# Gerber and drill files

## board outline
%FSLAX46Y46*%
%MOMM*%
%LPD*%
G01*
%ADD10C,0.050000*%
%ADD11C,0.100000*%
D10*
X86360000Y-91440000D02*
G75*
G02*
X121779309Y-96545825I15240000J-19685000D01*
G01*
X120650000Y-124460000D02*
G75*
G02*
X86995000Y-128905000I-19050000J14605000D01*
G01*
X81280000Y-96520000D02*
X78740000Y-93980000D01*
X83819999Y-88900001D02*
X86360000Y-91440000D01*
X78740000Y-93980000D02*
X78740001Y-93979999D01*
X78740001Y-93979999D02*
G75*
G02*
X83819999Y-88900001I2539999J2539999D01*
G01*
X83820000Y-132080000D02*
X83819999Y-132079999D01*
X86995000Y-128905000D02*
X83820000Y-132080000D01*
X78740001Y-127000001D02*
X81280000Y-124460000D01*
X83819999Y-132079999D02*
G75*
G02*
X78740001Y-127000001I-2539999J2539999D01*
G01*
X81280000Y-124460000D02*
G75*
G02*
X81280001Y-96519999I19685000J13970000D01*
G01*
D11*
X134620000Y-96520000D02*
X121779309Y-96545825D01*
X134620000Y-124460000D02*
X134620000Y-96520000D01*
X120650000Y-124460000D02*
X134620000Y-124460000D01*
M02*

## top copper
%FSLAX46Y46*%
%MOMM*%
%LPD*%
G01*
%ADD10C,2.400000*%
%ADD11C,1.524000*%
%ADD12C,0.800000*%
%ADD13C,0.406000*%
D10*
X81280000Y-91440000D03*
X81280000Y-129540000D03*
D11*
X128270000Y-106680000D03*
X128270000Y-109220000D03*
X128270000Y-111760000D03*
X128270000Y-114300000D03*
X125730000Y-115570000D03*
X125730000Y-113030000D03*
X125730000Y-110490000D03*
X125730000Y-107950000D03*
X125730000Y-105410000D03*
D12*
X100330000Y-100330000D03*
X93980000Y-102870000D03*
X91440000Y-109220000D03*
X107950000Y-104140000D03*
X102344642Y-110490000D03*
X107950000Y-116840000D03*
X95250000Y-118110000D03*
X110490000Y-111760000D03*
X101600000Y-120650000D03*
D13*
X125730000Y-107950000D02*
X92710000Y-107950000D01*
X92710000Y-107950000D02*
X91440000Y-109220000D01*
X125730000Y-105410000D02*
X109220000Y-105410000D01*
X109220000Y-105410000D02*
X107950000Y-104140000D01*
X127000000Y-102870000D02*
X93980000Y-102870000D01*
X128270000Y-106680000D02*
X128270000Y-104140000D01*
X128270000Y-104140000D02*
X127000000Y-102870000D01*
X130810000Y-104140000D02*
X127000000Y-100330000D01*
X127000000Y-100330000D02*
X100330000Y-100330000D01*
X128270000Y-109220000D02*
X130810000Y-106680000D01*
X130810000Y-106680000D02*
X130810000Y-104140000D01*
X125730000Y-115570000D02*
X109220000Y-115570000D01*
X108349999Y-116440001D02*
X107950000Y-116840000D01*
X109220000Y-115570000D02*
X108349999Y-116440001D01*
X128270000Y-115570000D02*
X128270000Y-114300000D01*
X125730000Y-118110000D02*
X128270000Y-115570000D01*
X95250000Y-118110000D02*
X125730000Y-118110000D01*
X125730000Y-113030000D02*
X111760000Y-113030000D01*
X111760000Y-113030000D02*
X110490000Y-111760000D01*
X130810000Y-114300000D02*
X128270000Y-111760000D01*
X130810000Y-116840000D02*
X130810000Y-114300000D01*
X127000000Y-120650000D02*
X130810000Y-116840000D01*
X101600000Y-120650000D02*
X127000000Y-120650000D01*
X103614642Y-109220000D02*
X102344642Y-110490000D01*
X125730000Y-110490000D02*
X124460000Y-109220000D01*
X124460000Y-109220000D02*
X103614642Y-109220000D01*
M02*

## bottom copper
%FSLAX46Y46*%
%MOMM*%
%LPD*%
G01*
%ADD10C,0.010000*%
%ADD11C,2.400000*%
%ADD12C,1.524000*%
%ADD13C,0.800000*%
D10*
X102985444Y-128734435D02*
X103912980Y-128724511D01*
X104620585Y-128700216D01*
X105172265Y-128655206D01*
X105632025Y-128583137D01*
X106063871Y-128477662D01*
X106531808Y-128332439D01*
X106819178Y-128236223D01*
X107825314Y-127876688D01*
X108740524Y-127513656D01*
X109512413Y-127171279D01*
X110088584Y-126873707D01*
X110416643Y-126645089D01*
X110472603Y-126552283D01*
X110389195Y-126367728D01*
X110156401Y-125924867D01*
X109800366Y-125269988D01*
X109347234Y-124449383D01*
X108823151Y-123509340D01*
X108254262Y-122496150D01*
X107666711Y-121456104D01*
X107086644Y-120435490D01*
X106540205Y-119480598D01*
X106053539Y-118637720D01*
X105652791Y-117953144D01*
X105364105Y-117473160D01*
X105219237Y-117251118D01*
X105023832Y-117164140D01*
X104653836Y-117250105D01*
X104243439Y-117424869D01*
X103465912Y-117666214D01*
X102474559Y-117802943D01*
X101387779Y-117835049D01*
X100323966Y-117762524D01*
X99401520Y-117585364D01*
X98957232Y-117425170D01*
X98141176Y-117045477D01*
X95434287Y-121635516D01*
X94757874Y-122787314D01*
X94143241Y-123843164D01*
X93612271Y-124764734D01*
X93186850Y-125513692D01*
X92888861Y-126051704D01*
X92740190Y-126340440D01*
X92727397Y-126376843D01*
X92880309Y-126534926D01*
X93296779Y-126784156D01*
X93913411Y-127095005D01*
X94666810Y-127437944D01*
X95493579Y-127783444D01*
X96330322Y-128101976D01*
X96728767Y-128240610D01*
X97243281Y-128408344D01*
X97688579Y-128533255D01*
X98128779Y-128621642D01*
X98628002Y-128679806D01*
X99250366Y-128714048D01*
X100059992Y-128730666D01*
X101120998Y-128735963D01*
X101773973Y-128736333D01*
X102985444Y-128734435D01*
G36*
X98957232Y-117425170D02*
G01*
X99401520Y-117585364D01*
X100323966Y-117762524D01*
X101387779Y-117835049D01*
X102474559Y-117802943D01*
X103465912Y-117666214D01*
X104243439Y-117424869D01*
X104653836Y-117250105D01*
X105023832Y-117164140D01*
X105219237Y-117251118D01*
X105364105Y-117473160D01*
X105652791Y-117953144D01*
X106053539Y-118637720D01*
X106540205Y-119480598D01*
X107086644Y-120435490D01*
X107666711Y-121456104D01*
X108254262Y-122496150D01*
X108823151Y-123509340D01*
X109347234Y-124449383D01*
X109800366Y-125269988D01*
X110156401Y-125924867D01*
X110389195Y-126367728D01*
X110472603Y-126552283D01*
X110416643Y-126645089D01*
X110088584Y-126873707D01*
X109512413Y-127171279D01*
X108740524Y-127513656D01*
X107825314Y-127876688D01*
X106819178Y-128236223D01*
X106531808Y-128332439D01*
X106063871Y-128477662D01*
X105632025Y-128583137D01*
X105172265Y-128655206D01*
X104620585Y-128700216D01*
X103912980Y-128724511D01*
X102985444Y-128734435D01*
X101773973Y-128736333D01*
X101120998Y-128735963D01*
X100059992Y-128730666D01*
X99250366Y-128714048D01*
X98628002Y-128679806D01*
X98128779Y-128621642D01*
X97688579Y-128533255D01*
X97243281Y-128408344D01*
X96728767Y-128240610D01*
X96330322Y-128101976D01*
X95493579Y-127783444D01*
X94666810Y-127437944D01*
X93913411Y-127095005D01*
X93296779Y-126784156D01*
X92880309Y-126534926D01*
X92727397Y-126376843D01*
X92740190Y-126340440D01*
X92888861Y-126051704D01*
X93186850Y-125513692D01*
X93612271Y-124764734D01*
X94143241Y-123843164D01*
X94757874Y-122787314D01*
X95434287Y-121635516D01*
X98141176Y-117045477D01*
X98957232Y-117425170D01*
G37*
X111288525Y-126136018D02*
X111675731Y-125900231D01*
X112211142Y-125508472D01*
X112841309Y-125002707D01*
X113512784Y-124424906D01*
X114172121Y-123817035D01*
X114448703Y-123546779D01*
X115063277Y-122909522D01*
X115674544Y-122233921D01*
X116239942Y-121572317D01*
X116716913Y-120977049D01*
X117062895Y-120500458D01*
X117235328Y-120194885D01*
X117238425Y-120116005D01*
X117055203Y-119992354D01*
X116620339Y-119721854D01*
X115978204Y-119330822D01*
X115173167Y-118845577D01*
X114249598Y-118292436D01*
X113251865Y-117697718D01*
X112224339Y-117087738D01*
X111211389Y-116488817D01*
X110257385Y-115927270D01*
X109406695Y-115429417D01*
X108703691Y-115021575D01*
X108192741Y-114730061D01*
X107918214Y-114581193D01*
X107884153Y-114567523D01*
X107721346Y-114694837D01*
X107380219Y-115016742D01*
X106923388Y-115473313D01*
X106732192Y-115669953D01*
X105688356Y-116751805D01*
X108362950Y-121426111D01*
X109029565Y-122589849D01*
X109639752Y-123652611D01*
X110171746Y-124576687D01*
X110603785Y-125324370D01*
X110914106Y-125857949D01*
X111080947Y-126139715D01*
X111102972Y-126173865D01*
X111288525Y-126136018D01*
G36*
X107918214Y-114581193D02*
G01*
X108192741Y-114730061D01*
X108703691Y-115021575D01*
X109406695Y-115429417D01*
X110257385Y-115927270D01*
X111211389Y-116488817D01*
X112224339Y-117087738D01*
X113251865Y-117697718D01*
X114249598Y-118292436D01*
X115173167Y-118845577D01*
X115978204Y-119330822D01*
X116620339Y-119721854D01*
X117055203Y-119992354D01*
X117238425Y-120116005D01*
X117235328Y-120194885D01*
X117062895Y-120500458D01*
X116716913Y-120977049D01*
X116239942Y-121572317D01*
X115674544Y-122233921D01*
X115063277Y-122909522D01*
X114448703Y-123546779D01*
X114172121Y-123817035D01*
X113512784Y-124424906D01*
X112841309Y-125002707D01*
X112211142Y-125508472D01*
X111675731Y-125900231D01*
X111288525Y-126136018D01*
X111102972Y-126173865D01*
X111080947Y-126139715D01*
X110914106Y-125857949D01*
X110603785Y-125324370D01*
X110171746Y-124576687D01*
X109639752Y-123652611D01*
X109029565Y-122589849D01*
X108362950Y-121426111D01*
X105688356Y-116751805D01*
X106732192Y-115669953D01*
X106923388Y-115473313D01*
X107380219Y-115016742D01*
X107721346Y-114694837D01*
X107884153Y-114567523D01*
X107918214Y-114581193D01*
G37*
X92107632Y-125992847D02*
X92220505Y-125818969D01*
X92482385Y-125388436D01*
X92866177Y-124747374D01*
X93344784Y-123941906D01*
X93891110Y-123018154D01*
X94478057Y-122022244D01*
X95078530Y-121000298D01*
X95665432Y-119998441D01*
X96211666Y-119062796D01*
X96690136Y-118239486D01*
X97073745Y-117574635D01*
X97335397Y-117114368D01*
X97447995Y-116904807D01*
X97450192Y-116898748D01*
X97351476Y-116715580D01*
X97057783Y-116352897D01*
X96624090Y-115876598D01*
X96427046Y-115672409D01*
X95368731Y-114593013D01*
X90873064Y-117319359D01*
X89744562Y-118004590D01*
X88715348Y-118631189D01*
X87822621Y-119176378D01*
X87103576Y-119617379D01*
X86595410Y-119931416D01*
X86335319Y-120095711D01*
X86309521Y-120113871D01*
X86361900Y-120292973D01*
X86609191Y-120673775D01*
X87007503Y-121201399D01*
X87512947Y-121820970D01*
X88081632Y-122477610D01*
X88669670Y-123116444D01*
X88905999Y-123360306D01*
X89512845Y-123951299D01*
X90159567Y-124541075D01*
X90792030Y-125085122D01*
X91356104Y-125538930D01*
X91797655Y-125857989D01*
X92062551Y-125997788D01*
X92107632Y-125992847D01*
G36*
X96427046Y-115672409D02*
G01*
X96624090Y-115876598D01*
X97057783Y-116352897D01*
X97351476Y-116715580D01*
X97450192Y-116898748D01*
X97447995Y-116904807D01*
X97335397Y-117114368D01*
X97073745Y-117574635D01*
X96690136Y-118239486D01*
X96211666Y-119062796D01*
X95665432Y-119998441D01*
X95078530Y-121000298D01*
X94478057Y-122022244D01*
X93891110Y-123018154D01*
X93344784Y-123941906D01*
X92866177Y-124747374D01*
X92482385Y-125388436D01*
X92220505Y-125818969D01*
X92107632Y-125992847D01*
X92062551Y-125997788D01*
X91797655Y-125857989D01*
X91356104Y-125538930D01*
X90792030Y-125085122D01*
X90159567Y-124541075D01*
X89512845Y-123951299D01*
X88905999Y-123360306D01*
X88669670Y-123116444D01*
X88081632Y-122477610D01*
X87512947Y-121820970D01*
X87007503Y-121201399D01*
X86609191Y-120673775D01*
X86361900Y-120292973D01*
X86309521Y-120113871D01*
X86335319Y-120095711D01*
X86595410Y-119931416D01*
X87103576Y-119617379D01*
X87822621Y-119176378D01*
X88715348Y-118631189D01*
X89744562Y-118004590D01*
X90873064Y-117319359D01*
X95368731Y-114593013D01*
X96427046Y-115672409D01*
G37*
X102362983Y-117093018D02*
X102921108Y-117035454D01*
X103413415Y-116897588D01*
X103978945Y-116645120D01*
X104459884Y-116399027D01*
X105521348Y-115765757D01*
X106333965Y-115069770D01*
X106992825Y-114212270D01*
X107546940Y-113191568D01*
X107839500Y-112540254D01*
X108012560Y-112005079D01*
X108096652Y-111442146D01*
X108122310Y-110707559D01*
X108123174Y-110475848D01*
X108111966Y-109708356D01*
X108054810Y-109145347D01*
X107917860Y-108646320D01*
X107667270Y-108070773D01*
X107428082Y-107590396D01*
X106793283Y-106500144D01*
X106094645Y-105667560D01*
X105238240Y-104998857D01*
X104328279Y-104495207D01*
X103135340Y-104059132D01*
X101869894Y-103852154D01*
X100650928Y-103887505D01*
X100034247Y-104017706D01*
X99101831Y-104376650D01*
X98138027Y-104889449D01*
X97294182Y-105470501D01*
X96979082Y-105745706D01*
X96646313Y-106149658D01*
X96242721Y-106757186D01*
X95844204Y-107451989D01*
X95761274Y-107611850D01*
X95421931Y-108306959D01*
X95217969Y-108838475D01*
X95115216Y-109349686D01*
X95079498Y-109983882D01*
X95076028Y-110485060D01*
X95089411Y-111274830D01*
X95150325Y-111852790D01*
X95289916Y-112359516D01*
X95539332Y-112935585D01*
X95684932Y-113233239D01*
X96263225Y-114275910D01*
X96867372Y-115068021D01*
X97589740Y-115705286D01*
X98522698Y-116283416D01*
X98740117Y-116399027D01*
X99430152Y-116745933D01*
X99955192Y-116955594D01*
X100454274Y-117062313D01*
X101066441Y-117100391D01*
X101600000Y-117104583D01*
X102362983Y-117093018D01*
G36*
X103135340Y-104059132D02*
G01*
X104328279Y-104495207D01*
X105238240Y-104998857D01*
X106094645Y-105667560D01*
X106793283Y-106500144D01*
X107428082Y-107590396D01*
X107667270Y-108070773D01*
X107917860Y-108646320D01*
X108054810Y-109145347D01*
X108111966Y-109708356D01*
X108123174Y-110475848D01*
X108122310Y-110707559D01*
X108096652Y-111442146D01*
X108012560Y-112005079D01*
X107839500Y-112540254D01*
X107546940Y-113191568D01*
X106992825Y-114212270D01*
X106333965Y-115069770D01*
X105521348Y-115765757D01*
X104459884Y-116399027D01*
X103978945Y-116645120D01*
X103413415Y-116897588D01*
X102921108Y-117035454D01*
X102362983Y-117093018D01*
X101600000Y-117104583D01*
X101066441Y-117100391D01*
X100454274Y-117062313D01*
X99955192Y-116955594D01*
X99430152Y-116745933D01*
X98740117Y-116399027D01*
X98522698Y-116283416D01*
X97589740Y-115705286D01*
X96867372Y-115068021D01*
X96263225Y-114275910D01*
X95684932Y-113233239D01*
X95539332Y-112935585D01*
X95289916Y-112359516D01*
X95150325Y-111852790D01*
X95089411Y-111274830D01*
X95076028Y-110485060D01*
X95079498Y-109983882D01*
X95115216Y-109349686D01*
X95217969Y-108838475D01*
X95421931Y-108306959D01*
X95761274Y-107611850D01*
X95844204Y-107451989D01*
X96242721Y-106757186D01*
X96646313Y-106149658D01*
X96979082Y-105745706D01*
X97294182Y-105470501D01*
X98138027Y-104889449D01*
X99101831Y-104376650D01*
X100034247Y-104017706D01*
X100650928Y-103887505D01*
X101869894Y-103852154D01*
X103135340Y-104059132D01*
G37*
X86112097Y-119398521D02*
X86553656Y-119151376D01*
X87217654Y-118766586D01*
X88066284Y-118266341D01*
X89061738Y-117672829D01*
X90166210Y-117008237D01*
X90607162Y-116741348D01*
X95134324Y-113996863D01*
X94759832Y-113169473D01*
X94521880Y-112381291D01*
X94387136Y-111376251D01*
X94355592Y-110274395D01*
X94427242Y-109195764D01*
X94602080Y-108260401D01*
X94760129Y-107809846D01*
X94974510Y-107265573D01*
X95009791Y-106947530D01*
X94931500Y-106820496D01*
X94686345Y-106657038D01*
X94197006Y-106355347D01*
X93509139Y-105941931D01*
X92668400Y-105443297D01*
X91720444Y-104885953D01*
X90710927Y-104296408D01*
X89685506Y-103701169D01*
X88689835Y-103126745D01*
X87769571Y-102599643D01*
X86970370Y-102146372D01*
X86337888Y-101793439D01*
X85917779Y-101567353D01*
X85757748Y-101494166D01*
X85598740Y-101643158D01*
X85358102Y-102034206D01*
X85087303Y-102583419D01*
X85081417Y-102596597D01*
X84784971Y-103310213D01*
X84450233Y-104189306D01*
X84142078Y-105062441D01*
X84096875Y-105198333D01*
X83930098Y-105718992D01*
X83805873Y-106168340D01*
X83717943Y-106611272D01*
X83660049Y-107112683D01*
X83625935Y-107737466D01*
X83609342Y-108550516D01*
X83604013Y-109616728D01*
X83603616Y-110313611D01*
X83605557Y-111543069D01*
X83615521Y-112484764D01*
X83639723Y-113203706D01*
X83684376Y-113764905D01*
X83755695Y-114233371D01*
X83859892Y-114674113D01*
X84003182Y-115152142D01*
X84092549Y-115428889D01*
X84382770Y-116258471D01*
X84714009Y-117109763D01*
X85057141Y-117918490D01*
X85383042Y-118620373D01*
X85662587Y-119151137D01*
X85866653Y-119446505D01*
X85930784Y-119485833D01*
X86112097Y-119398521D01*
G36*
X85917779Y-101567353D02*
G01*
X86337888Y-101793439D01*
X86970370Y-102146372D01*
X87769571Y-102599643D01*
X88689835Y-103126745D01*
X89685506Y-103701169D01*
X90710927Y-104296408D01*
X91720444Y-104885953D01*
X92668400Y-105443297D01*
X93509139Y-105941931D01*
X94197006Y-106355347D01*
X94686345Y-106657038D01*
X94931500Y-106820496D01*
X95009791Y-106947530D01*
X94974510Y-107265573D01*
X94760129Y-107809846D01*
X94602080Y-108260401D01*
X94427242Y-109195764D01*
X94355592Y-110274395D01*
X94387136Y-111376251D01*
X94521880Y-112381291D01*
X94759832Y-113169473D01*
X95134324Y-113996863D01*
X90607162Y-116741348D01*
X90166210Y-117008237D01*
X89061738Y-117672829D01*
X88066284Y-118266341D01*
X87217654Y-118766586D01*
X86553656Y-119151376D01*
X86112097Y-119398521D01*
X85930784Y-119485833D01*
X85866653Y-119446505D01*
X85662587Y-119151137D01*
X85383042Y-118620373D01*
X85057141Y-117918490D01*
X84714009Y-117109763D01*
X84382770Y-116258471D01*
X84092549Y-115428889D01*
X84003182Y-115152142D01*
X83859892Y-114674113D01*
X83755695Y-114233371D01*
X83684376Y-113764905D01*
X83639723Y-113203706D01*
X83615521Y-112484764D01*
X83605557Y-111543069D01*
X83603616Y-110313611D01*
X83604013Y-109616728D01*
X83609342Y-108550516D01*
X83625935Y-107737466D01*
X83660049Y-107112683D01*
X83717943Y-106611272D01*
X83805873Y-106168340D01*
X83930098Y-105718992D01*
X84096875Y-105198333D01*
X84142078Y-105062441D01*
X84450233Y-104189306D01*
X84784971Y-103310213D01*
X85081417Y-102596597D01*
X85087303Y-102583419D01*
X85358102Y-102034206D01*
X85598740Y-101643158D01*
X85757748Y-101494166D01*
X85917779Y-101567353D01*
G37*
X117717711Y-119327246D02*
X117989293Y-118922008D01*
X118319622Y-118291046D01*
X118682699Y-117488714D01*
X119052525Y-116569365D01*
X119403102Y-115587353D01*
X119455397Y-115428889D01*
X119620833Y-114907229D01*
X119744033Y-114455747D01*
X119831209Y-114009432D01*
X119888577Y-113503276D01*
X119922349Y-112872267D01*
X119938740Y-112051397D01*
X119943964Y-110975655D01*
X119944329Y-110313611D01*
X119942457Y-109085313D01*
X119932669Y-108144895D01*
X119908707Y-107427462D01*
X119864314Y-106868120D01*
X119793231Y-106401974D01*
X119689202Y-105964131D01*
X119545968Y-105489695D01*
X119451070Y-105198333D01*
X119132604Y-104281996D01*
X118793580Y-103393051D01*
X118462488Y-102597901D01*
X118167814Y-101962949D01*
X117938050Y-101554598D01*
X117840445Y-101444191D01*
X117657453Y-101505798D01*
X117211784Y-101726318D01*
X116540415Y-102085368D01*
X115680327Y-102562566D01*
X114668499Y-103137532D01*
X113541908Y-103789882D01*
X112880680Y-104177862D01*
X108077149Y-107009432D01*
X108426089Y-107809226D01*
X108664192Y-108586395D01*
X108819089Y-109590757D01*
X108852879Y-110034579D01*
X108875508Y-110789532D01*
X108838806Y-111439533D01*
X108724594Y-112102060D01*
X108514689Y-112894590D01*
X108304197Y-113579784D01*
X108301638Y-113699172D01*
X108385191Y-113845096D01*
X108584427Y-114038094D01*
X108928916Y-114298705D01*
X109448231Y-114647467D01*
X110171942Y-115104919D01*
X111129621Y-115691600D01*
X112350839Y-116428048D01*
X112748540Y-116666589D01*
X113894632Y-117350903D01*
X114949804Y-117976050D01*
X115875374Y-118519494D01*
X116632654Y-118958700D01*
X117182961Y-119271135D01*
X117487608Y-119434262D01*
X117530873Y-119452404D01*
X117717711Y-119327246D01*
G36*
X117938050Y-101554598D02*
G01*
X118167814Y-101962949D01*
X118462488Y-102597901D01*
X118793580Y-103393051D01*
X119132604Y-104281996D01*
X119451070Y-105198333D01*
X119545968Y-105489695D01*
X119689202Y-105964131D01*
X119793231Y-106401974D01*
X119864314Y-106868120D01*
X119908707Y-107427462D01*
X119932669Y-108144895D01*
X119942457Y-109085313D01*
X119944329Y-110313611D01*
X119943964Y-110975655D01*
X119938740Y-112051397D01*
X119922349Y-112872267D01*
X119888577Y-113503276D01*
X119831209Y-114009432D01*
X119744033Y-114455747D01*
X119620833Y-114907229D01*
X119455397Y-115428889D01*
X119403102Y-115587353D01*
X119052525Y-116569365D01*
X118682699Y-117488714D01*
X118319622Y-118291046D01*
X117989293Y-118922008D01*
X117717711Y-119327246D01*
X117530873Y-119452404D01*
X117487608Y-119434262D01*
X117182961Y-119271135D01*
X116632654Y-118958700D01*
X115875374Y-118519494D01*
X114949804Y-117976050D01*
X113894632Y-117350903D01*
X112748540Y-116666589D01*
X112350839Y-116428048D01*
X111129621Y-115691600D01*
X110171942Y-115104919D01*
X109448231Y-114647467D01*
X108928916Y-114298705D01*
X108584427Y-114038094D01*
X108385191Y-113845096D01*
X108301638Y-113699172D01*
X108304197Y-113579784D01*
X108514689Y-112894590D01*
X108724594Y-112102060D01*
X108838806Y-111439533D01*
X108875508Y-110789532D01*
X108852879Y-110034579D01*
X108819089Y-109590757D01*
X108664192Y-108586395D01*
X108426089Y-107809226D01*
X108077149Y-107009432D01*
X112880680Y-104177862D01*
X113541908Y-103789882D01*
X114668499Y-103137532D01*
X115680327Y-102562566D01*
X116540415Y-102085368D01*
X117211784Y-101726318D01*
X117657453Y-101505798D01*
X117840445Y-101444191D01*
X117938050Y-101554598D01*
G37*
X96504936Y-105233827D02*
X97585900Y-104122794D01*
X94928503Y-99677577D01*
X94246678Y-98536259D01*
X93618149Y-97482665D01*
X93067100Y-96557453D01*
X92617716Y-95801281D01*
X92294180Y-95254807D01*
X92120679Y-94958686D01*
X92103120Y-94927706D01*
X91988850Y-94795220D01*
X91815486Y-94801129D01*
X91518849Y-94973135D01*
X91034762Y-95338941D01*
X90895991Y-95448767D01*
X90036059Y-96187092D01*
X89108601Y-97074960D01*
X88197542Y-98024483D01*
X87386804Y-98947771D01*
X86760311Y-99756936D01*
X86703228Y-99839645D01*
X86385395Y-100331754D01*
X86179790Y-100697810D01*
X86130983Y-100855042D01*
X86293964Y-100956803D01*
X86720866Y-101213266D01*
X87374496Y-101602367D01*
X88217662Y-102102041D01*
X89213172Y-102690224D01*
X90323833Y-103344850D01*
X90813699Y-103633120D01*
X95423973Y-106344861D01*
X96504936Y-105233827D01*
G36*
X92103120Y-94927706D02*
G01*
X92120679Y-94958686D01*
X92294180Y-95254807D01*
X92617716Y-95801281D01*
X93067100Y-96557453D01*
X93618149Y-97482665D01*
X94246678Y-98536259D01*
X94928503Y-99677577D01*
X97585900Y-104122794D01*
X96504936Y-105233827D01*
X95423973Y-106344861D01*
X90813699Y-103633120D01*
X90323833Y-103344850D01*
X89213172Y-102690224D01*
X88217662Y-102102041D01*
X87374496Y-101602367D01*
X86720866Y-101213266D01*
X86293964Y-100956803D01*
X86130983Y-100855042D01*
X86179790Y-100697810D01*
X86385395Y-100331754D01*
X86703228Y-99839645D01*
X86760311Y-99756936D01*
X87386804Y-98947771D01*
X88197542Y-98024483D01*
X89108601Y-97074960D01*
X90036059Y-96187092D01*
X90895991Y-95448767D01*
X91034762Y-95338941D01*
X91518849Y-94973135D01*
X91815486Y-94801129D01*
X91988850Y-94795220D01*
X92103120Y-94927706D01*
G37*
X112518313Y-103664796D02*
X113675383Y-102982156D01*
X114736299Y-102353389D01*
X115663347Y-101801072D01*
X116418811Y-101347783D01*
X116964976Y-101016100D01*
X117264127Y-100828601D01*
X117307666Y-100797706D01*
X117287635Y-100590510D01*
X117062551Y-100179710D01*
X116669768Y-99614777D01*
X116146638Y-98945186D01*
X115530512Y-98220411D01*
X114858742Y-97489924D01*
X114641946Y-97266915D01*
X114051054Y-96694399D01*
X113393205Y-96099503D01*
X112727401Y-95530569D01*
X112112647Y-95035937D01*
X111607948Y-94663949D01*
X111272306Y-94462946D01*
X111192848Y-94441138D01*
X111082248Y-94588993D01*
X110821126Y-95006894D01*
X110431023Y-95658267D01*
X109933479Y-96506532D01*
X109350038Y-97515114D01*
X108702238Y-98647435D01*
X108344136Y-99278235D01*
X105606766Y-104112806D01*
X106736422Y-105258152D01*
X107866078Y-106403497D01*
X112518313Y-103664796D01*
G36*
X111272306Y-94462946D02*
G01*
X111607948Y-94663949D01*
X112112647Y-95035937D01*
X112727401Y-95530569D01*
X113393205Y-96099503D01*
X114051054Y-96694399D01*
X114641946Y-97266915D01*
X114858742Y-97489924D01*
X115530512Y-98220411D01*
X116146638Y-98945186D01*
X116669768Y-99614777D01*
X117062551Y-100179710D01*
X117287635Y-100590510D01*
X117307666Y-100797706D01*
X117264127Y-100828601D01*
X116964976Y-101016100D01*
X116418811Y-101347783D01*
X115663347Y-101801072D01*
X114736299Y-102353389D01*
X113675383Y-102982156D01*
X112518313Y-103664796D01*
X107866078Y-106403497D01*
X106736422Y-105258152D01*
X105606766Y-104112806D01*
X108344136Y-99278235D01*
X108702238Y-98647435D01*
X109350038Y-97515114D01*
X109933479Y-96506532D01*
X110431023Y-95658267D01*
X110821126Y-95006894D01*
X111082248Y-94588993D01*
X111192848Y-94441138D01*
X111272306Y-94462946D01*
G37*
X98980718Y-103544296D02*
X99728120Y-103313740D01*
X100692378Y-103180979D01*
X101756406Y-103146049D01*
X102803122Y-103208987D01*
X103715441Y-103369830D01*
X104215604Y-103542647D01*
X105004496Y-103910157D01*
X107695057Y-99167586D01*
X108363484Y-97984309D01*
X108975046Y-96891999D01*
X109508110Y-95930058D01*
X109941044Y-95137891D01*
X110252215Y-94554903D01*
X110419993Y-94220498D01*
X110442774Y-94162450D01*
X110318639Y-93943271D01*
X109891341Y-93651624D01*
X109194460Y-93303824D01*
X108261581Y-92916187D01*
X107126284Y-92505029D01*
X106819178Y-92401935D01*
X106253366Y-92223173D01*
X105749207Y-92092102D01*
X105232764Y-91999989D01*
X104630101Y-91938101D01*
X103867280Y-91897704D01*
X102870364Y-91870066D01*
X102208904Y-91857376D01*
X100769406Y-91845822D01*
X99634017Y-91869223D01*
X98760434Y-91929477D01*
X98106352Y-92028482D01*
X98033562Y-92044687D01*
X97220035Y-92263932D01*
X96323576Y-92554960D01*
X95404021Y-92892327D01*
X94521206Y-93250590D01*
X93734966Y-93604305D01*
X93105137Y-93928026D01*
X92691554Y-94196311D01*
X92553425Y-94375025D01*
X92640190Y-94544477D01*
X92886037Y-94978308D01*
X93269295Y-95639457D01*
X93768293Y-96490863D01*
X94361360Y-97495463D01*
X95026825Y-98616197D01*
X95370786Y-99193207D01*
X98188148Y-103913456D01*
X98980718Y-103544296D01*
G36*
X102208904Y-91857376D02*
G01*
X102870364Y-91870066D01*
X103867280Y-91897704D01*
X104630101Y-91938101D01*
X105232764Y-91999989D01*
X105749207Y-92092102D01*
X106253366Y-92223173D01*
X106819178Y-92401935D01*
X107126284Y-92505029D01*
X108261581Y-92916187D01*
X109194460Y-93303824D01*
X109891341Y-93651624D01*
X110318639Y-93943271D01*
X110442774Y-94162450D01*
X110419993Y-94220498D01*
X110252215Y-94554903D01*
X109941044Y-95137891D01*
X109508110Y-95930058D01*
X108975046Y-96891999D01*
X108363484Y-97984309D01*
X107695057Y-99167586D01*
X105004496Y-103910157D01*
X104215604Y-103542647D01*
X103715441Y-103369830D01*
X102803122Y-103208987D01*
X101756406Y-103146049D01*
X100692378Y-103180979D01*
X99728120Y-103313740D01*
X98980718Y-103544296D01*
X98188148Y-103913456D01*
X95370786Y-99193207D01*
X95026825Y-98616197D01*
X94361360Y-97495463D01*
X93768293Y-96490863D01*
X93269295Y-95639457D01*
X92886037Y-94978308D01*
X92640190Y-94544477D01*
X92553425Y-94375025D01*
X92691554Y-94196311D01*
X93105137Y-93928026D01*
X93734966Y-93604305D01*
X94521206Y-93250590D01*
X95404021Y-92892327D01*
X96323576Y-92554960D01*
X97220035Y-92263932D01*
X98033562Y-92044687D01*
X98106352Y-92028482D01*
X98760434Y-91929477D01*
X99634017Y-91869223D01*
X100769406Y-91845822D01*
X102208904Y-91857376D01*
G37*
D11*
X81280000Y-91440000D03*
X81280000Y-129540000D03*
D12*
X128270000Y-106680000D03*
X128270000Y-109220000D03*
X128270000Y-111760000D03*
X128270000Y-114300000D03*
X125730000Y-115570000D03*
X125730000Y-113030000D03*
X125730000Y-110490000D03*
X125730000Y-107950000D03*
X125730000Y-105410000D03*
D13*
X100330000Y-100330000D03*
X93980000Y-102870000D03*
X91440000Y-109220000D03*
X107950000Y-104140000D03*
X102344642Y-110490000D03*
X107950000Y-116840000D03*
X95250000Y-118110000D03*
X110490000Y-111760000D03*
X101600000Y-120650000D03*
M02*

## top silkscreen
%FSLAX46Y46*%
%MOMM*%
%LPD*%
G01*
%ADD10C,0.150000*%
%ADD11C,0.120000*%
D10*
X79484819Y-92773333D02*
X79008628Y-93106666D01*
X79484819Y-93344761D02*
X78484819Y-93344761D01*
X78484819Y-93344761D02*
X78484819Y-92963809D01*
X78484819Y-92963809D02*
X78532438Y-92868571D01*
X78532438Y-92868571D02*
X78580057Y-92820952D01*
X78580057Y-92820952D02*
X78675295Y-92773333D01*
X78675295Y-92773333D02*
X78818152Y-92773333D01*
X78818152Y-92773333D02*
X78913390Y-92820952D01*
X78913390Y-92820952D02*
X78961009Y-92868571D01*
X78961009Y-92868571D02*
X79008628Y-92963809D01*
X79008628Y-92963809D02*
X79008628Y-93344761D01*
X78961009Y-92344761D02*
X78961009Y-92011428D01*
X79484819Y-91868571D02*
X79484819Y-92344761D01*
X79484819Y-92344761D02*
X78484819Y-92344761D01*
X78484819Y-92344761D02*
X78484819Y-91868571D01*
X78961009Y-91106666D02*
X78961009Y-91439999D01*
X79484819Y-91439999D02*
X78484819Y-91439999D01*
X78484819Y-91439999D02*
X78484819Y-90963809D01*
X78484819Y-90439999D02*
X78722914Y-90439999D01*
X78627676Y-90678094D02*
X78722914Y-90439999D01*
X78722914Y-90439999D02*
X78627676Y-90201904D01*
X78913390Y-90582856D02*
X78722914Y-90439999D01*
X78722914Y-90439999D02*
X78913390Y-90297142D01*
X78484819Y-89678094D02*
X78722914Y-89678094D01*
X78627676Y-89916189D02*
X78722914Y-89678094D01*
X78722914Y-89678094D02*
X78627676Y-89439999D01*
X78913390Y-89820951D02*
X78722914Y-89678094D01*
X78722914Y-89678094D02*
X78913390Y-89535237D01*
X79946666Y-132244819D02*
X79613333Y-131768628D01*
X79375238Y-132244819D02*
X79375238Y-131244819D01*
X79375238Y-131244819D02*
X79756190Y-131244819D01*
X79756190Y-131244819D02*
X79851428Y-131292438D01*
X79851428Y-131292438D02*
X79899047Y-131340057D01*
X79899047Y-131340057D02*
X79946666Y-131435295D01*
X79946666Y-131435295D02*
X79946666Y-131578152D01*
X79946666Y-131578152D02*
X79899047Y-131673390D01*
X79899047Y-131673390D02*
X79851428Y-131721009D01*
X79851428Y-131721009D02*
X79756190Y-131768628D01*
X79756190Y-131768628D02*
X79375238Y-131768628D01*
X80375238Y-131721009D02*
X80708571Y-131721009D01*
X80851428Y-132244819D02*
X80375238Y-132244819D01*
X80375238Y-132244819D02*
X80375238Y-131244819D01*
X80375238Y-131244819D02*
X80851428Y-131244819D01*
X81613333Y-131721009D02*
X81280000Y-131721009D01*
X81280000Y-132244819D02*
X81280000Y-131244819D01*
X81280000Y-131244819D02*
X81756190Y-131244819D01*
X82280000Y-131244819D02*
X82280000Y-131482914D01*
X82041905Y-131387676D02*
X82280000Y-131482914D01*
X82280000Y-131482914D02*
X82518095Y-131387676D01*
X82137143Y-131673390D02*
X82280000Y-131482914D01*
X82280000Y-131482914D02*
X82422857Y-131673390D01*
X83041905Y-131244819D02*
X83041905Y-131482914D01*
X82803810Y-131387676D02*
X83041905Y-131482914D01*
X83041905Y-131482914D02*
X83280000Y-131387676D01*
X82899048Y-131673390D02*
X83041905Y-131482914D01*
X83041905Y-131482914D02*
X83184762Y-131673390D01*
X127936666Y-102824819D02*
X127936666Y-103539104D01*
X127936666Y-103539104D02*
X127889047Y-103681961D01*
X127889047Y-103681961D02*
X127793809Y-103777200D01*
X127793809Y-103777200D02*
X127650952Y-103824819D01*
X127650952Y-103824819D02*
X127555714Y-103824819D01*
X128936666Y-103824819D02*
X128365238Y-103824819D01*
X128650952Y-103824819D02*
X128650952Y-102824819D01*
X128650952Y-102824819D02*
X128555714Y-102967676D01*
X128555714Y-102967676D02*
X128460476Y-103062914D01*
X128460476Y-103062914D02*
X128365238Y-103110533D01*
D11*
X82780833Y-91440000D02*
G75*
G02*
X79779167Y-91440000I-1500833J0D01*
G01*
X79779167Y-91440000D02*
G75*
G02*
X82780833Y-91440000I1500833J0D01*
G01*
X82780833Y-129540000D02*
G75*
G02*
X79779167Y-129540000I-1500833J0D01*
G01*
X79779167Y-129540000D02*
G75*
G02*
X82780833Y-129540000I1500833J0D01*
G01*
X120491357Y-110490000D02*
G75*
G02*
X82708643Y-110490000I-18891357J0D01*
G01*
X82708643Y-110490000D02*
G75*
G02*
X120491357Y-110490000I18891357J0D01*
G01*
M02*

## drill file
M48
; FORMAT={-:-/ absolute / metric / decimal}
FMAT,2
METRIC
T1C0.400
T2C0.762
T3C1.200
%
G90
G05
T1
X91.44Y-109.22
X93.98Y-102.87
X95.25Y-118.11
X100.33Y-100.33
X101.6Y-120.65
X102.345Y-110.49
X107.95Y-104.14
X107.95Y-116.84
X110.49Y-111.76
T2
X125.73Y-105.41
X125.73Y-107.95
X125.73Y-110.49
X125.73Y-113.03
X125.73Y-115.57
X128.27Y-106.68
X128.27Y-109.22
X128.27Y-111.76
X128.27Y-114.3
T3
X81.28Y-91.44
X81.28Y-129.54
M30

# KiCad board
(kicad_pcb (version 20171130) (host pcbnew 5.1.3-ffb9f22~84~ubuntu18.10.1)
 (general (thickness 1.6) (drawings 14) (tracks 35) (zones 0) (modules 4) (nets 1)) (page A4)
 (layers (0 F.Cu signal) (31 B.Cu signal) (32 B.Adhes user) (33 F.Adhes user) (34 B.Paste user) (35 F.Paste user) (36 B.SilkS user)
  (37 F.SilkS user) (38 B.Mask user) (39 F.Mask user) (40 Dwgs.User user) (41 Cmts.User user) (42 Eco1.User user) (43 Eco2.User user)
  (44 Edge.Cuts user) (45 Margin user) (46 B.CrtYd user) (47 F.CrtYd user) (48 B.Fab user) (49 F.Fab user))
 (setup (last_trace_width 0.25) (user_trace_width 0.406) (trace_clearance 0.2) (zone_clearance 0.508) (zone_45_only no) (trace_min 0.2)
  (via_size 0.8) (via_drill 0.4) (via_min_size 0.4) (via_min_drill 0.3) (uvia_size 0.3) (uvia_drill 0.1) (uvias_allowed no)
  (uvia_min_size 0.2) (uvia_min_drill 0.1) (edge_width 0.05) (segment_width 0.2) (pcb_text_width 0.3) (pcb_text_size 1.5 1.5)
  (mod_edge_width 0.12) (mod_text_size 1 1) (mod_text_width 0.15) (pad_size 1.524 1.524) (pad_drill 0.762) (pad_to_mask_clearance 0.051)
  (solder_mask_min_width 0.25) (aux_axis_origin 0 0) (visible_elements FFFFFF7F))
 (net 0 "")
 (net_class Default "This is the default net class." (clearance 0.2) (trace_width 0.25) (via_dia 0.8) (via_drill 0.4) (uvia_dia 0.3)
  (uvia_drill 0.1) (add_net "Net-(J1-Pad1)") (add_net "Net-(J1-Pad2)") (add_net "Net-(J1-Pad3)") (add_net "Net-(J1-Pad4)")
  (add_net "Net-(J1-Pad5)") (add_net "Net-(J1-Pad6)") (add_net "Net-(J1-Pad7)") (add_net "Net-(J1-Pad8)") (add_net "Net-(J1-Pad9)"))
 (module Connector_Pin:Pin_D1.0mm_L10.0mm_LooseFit (layer F.Cu) (at 81.28 91.44 270)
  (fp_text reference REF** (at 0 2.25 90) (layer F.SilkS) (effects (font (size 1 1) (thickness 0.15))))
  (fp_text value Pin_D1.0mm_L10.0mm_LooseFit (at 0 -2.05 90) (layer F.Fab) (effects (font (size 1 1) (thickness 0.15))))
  (fp_circle (center 0 0) (end 1.5 0.05) (layer F.SilkS) (width 0.12))
  (pad 1 thru_hole circle (at 0 0 270) (size 2.4 2.4) (drill 1.2) (layers *.Cu *.Mask)))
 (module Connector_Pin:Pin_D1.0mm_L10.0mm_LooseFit (layer F.Cu) (at 81.28 129.54)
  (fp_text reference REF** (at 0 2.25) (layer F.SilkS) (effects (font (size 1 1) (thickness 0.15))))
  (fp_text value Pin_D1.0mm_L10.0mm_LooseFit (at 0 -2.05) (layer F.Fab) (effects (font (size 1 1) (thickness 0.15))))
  (fp_circle (center 0 0) (end 1.5 0.05) (layer F.SilkS) (width 0.12))
  (pad 1 thru_hole circle (at 0 0) (size 2.4 2.4) (drill 1.2) (layers *.Cu *.Mask)))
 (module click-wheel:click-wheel (layer B.Cu) (at 101.6 110.49)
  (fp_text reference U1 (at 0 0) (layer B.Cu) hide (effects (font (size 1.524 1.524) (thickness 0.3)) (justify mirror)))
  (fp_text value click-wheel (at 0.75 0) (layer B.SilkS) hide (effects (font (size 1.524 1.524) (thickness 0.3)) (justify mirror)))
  (fp_circle (center 0 0) (end 16.51 -9.181682) (layer F.SilkS) (width 0.12))
  (fp_poly
   (pts (xy 1.385444 18.244435) (xy 2.31298 18.234511) (xy 3.020585 18.210216) (xy 3.572265 18.165206) (xy 4.032025 18.093137)
    (xy 4.463871 17.987662) (xy 4.931808 17.842439) (xy 5.219178 17.746223) (xy 6.225314 17.386688) (xy 7.140524 17.023656)
    (xy 7.912413 16.681279) (xy 8.488584 16.383707) (xy 8.816643 16.155089) (xy 8.872603 16.062283) (xy 8.789195 15.877728)
    (xy 8.556401 15.434867) (xy 8.200366 14.779988) (xy 7.747234 13.959383) (xy 7.223151 13.01934) (xy 6.654262 12.00615)
    (xy 6.066711 10.966104) (xy 5.486644 9.94549) (xy 4.940205 8.990598) (xy 4.453539 8.14772) (xy 4.052791 7.463144) (xy 3.764105 6.98316)
    (xy 3.619237 6.761118) (xy 3.423832 6.67414) (xy 3.053836 6.760105) (xy 2.643439 6.934869) (xy 1.865912 7.176214) (xy 0.874559 7.312943)
    (xy -0.212221 7.345049) (xy -1.276034 7.272524) (xy -2.19848 7.095364) (xy -2.642768 6.93517) (xy -3.458824 6.555477)
    (xy -6.165713 11.145516) (xy -6.842126 12.297314) (xy -7.456759 13.353164) (xy -7.987729 14.274734) (xy -8.41315 15.023692)
    (xy -8.711139 15.561704) (xy -8.85981 15.85044) (xy -8.872603 15.886843) (xy -8.719691 16.044926) (xy -8.303221 16.294156)
    (xy -7.686589 16.605005) (xy -6.93319 16.947944) (xy -6.106421 17.293444) (xy -5.269678 17.611976) (xy -4.871233 17.75061)
    (xy -4.356719 17.918344) (xy -3.911421 18.043255) (xy -3.471221 18.131642) (xy -2.971998 18.189806) (xy -2.349634 18.224048)
    (xy -1.540008 18.240666) (xy -0.479002 18.245963) (xy 0.173973 18.246333) (xy 1.385444 18.244435))
   (layer B.Cu) (width 0.01))
  (fp_poly
   (pts (xy 9.688525 15.646018) (xy 10.075731 15.410231) (xy 10.611142 15.018472) (xy 11.241309 14.512707) (xy 11.912784 13.934906)
    (xy 12.572121 13.327035) (xy 12.848703 13.056779) (xy 13.463277 12.419522) (xy 14.074544 11.743921) (xy 14.639942 11.082317)
    (xy 15.116913 10.487049) (xy 15.462895 10.010458) (xy 15.635328 9.704885) (xy 15.638425 9.626005) (xy 15.455203 9.502354)
    (xy 15.020339 9.231854) (xy 14.378204 8.840822) (xy 13.573167 8.355577) (xy 12.649598 7.802436) (xy 11.651865 7.207718)
    (xy 10.624339 6.597738) (xy 9.611389 5.998817) (xy 8.657385 5.43727) (xy 7.806695 4.939417) (xy 7.103691 4.531575)
    (xy 6.592741 4.240061) (xy 6.318214 4.091193) (xy 6.284153 4.077523) (xy 6.121346 4.204837) (xy 5.780219 4.526742)
    (xy 5.323388 4.983313) (xy 5.132192 5.179953) (xy 4.088356 6.261805) (xy 6.76295 10.936111) (xy 7.429565 12.099849)
    (xy 8.039752 13.162611) (xy 8.571746 14.086687) (xy 9.003785 14.83437) (xy 9.314106 15.367949) (xy 9.480947 15.649715)
    (xy 9.502972 15.683865) (xy 9.688525 15.646018))
   (layer B.Cu) (width 0.01))
  (fp_poly
   (pts (xy -9.492368 15.502847) (xy -9.379495 15.328969) (xy -9.117615 14.898436) (xy -8.733823 14.257374) (xy -8.255216 13.451906)
    (xy -7.70889 12.528154) (xy -7.121943 11.532244) (xy -6.52147 10.510298) (xy -5.934568 9.508441) (xy -5.388334 8.572796)
    (xy -4.909864 7.749486) (xy -4.526255 7.084635) (xy -4.264603 6.624368) (xy -4.152005 6.414807) (xy -4.149808 6.408748)
    (xy -4.248524 6.22558) (xy -4.542217 5.862897) (xy -4.97591 5.386598) (xy -5.172954 5.182409) (xy -6.231269 4.103013)
    (xy -10.726936 6.829359) (xy -11.855438 7.51459) (xy -12.884652 8.141189) (xy -13.777379 8.686378) (xy -14.496424 9.127379)
    (xy -15.00459 9.441416) (xy -15.264681 9.605711) (xy -15.290479 9.623871) (xy -15.2381 9.802973) (xy -14.990809 10.183775)
    (xy -14.592497 10.711399) (xy -14.087053 11.33097) (xy -13.518368 11.98761) (xy -12.93033 12.626444) (xy -12.694001 12.870306)
    (xy -12.087155 13.461299) (xy -11.440433 14.051075) (xy -10.80797 14.595122) (xy -10.243896 15.04893) (xy -9.802345 15.367989)
    (xy -9.537449 15.507788) (xy -9.492368 15.502847))
   (layer B.Cu) (width 0.01))
  (fp_poly
   (pts (xy 0.762983 6.603018) (xy 1.321108 6.545454) (xy 1.813415 6.407588) (xy 2.378945 6.15512) (xy 2.859884 5.909027)
    (xy 3.921348 5.275757) (xy 4.733965 4.57977) (xy 5.392825 3.72227) (xy 5.94694 2.701568) (xy 6.2395 2.050254) (xy 6.41256 1.515079)
    (xy 6.496652 0.952146) (xy 6.52231 0.217559) (xy 6.523174 -0.014152) (xy 6.511966 -0.781644) (xy 6.45481 -1.344653)
    (xy 6.31786 -1.84368) (xy 6.06727 -2.419227) (xy 5.828082 -2.899604) (xy 5.193283 -3.989856) (xy 4.494645 -4.82244)
    (xy 3.63824 -5.491143) (xy 2.728279 -5.994793) (xy 1.53534 -6.430868) (xy 0.269894 -6.637846) (xy -0.949072 -6.602495)
    (xy -1.565753 -6.472294) (xy -2.498169 -6.11335) (xy -3.461973 -5.600551) (xy -4.305818 -5.019499) (xy -4.620918 -4.744294)
    (xy -4.953687 -4.340342) (xy -5.357279 -3.732814) (xy -5.755796 -3.038011) (xy -5.838726 -2.87815) (xy -6.178069 -2.183041)
    (xy -6.382031 -1.651525) (xy -6.484784 -1.140314) (xy -6.520502 -0.506118) (xy -6.523972 -0.00494) (xy -6.510589 0.78483)
    (xy -6.449675 1.36279) (xy -6.310084 1.869516) (xy -6.060668 2.445585) (xy -5.915068 2.743239) (xy -5.336775 3.78591)
    (xy -4.732628 4.578021) (xy -4.01026 5.215286) (xy -3.077302 5.793416) (xy -2.859883 5.909027) (xy -2.169848 6.255933)
    (xy -1.644808 6.465594) (xy -1.145726 6.572313) (xy -0.533559 6.610391) (xy 0 6.614583) (xy 0.762983 6.603018))
   (layer B.Cu) (width 0.01))
  (fp_poly
   (pts (xy -15.487903 8.908521) (xy -15.046344 8.661376) (xy -14.382346 8.276586) (xy -13.533716 7.776341) (xy -12.538262 7.182829)
    (xy -11.43379 6.518237) (xy -10.992838 6.251348) (xy -6.465676 3.506863) (xy -6.840168 2.679473) (xy -7.07812 1.891291)
    (xy -7.212864 0.886251) (xy -7.244408 -0.215605) (xy -7.172758 -1.294236) (xy -6.99792 -2.229599) (xy -6.839871 -2.680154)
    (xy -6.62549 -3.224427) (xy -6.590209 -3.54247) (xy -6.6685 -3.669504) (xy -6.913655 -3.832962) (xy -7.402994 -4.134653)
    (xy -8.090861 -4.548069) (xy -8.9316 -5.046703) (xy -9.879556 -5.604047) (xy -10.889073 -6.193592) (xy -11.914494 -6.788831)
    (xy -12.910165 -7.363255) (xy -13.830429 -7.890357) (xy -14.62963 -8.343628) (xy -15.262112 -8.696561) (xy -15.682221 -8.922647)
    (xy -15.842252 -8.995834) (xy -16.00126 -8.846842) (xy -16.241898 -8.455794) (xy -16.512697 -7.906581) (xy -16.518583 -7.893403)
    (xy -16.815029 -7.179787) (xy -17.149767 -6.300694) (xy -17.457922 -5.427559) (xy -17.503125 -5.291667) (xy -17.669902 -4.771008)
    (xy -17.794127 -4.32166) (xy -17.882057 -3.878728) (xy -17.939951 -3.377317) (xy -17.974065 -2.752534) (xy -17.990658 -1.939484)
    (xy -17.995987 -0.873272) (xy -17.996384 -0.176389) (xy -17.994443 1.053069) (xy -17.984479 1.994764) (xy -17.960277 2.713706)
    (xy -17.915624 3.274905) (xy -17.844305 3.743371) (xy -17.740108 4.184113) (xy -17.596818 4.662142) (xy -17.507451 4.938889)
    (xy -17.21723 5.768471) (xy -16.885991 6.619763) (xy -16.542859 7.42849) (xy -16.216958 8.130373) (xy -15.937413 8.661137)
    (xy -15.733347 8.956505) (xy -15.669216 8.995833) (xy -15.487903 8.908521))
   (layer B.Cu) (width 0.01))
  (fp_poly
   (pts (xy 16.117711 8.837246) (xy 16.389293 8.432008) (xy 16.719622 7.801046) (xy 17.082699 6.998714) (xy 17.452525 6.079365)
    (xy 17.803102 5.097353) (xy 17.855397 4.938889) (xy 18.020833 4.417229) (xy 18.144033 3.965747) (xy 18.231209 3.519432)
    (xy 18.288577 3.013276) (xy 18.322349 2.382267) (xy 18.33874 1.561397) (xy 18.343964 0.485655) (xy 18.344329 -0.176389)
    (xy 18.342457 -1.404687) (xy 18.332669 -2.345105) (xy 18.308707 -3.062538) (xy 18.264314 -3.62188) (xy 18.193231 -4.088026)
    (xy 18.089202 -4.525869) (xy 17.945968 -5.000305) (xy 17.85107 -5.291667) (xy 17.532604 -6.208004) (xy 17.19358 -7.096949)
    (xy 16.862488 -7.892099) (xy 16.567814 -8.527051) (xy 16.33805 -8.935402) (xy 16.240445 -9.045809) (xy 16.057453 -8.984202)
    (xy 15.611784 -8.763682) (xy 14.940415 -8.404632) (xy 14.080327 -7.927434) (xy 13.068499 -7.352468) (xy 11.941908 -6.700118)
    (xy 11.28068 -6.312138) (xy 6.477149 -3.480568) (xy 6.826089 -2.680774) (xy 7.064192 -1.903605) (xy 7.219089 -0.899243)
    (xy 7.252879 -0.455421) (xy 7.275508 0.299532) (xy 7.238806 0.949533) (xy 7.124594 1.61206) (xy 6.914689 2.40459) (xy 6.704197 3.089784)
    (xy 6.701638 3.209172) (xy 6.785191 3.355096) (xy 6.984427 3.548094) (xy 7.328916 3.808705) (xy 7.848231 4.157467)
    (xy 8.571942 4.614919) (xy 9.529621 5.2016) (xy 10.750839 5.938048) (xy 11.14854 6.176589) (xy 12.294632 6.860903)
    (xy 13.349804 7.48605) (xy 14.275374 8.029494) (xy 15.032654 8.4687) (xy 15.582961 8.781135) (xy 15.887608 8.944262)
    (xy 15.930873 8.962404) (xy 16.117711 8.837246))
   (layer B.Cu) (width 0.01))
  (fp_poly
   (pts (xy -5.095064 -5.256173) (xy -4.0141 -6.367206) (xy -6.671497 -10.812423) (xy -7.353322 -11.953741) (xy -7.981851 -13.007335)
    (xy -8.5329 -13.932547) (xy -8.982284 -14.688719) (xy -9.30582 -15.235193) (xy -9.479321 -15.531314) (xy -9.49688 -15.562294)
    (xy -9.61115 -15.69478) (xy -9.784514 -15.688871) (xy -10.081151 -15.516865) (xy -10.565238 -15.151059) (xy -10.704009 -15.041233)
    (xy -11.563941 -14.302908) (xy -12.491399 -13.41504) (xy -13.402458 -12.465517) (xy -14.213196 -11.542229) (xy -14.839689 -10.733064)
    (xy -14.896772 -10.650355) (xy -15.214605 -10.158246) (xy -15.42021 -9.79219) (xy -15.469017 -9.634958) (xy -15.306036 -9.533197)
    (xy -14.879134 -9.276734) (xy -14.225504 -8.887633) (xy -13.382338 -8.387959) (xy -12.386828 -7.799776) (xy -11.276167 -7.14515)
    (xy -10.786301 -6.85688) (xy -6.176027 -4.145139) (xy -5.095064 -5.256173))
   (layer B.Cu) (width 0.01))
  (fp_poly
   (pts (xy 10.918313 -6.825204) (xy 12.075383 -7.507844) (xy 13.136299 -8.136611) (xy 14.063347 -8.688928) (xy 14.818811 -9.142217)
    (xy 15.364976 -9.4739) (xy 15.664127 -9.661399) (xy 15.707666 -9.692294) (xy 15.687635 -9.89949) (xy 15.462551 -10.31029)
    (xy 15.069768 -10.875223) (xy 14.546638 -11.544814) (xy 13.930512 -12.269589) (xy 13.258742 -13.000076) (xy 13.041946 -13.223085)
    (xy 12.451054 -13.795601) (xy 11.793205 -14.390497) (xy 11.127401 -14.959431) (xy 10.512647 -15.454063) (xy 10.007948 -15.826051)
    (xy 9.672306 -16.027054) (xy 9.592848 -16.048862) (xy 9.482248 -15.901007) (xy 9.221126 -15.483106) (xy 8.831023 -14.831733)
    (xy 8.333479 -13.983468) (xy 7.750038 -12.974886) (xy 7.102238 -11.842565) (xy 6.744136 -11.211765) (xy 4.006766 -6.377194)
    (xy 5.136422 -5.231848) (xy 6.266078 -4.086503) (xy 10.918313 -6.825204))
   (layer B.Cu) (width 0.01))
  (fp_poly
   (pts (xy -2.619282 -6.945704) (xy -1.87188 -7.17626) (xy -0.907622 -7.309021) (xy 0.156406 -7.343951) (xy 1.203122 -7.281013)
    (xy 2.115441 -7.12017) (xy 2.615604 -6.947353) (xy 3.404496 -6.579843) (xy 6.095057 -11.322414) (xy 6.763484 -12.505691)
    (xy 7.375046 -13.598001) (xy 7.90811 -14.559942) (xy 8.341044 -15.352109) (xy 8.652215 -15.935097) (xy 8.819993 -16.269502)
    (xy 8.842774 -16.32755) (xy 8.718639 -16.546729) (xy 8.291341 -16.838376) (xy 7.59446 -17.186176) (xy 6.661581 -17.573813)
    (xy 5.526284 -17.984971) (xy 5.219178 -18.088065) (xy 4.653366 -18.266827) (xy 4.149207 -18.397898) (xy 3.632764 -18.490011)
    (xy 3.030101 -18.551899) (xy 2.26728 -18.592296) (xy 1.270364 -18.619934) (xy 0.608904 -18.632624) (xy -0.830594 -18.644178)
    (xy -1.965983 -18.620777) (xy -2.839566 -18.560523) (xy -3.493648 -18.461518) (xy -3.566438 -18.445313) (xy -4.379965 -18.226068)
    (xy -5.276424 -17.93504) (xy -6.195979 -17.597673) (xy -7.078794 -17.23941) (xy -7.865034 -16.885695) (xy -8.494863 -16.561974)
    (xy -8.908446 -16.293689) (xy -9.046575 -16.114975) (xy -8.95981 -15.945523) (xy -8.713963 -15.511692) (xy -8.330705 -14.850543)
    (xy -7.831707 -13.999137) (xy -7.23864 -12.994537) (xy -6.573175 -11.873803) (xy -6.229214 -11.296793) (xy -3.411852 -6.576544)
    (xy -2.619282 -6.945704))
   (layer B.Cu) (width 0.01)))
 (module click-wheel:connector (layer F.Cu) (at 128.27 102.87)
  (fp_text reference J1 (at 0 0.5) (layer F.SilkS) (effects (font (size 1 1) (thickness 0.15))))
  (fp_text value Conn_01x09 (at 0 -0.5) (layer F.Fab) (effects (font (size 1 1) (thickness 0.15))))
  (pad 9 thru_hole circle (at 0 3.81) (size 1.524 1.524) (drill 0.762) (layers *.Cu *.Mask))
  (pad 8 thru_hole circle (at 0 6.35) (size 1.524 1.524) (drill 0.762) (layers *.Cu *.Mask))
  (pad 7 thru_hole circle (at 0 8.89) (size 1.524 1.524) (drill 0.762) (layers *.Cu *.Mask))
  (pad 6 thru_hole circle (at 0 11.43) (size 1.524 1.524) (drill 0.762) (layers *.Cu *.Mask))
  (pad 5 thru_hole circle (at -2.54 12.7) (size 1.524 1.524) (drill 0.762) (layers *.Cu *.Mask))
  (pad 4 thru_hole circle (at -2.54 10.16) (size 1.524 1.524) (drill 0.762) (layers *.Cu *.Mask))
  (pad 3 thru_hole circle (at -2.54 7.62) (size 1.524 1.524) (drill 0.762) (layers *.Cu *.Mask))
  (pad 2 thru_hole circle (at -2.54 5.08) (size 1.524 1.524) (drill 0.762) (layers *.Cu *.Mask))
  (pad 1 thru_hole circle (at -2.54 2.54) (size 1.524 1.524) (drill 0.762) (layers *.Cu *.Mask)))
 (gr_arc (start 101.6 111.125) (end 86.36 91.44) (angle 91.8993953) (layer Edge.Cuts) (width 0.05))
 (gr_arc (start 101.6 109.855) (end 120.65 124.46) (angle 90) (layer Edge.Cuts) (width 0.05))
 (gr_line (start 81.28 96.52) (end 78.74 93.98) (layer Edge.Cuts) (width 0.05))
 (gr_line (start 83.819999 88.900001) (end 86.36 91.44) (layer Edge.Cuts) (width 0.05))
 (gr_line (start 78.74 93.98) (end 78.740001 93.979999) (layer Edge.Cuts) (width 0.05))
 (gr_arc (start 81.28 91.44) (end 83.819999 88.900001) (angle -180) (layer Edge.Cuts) (width 0.05))
 (gr_line (start 83.82 132.08) (end 83.819999 132.079999) (layer Edge.Cuts) (width 0.05))
 (gr_line (start 86.995 128.905) (end 83.82 132.08) (layer Edge.Cuts) (width 0.05))
 (gr_line (start 78.740001 127.000001) (end 81.28 124.46) (layer Edge.Cuts) (width 0.05))
 (gr_arc (start 81.28 129.54) (end 78.740001 127.000001) (angle -180) (layer Edge.Cuts) (width 0.05))
 (gr_arc (start 100.965 110.49) (end 81.28 124.46) (angle 70.72492708) (layer Edge.Cuts) (width 0.05))
 (gr_line (start 134.62 96.52) (end 121.779309 96.545825) (layer Edge.Cuts) (width 0.1))
 (gr_line (start 134.62 124.46) (end 134.62 96.52) (layer Edge.Cuts) (width 0.1))
 (gr_line (start 120.65 124.46) (end 134.62 124.46) (layer Edge.Cuts) (width 0.1))
 (via (at 100.33 100.33) (size 0.8) (drill 0.4) (layers F.Cu B.Cu) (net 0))
 (via (at 93.98 102.87) (size 0.8) (drill 0.4) (layers F.Cu B.Cu) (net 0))
 (segment (start 125.73 107.95) (end 92.71 107.95) (width 0.406) (layer F.Cu) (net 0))
 (via (at 91.44 109.22) (size 0.8) (drill 0.4) (layers F.Cu B.Cu) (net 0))
 (segment (start 92.71 107.95) (end 91.44 109.22) (width 0.406) (layer F.Cu) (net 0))
 (via (at 107.95 104.14) (size 0.8) (drill 0.4) (layers F.Cu B.Cu) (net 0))
 (segment (start 125.73 105.41) (end 109.22 105.41) (width 0.406) (layer F.Cu) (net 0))
 (segment (start 109.22 105.41) (end 107.95 104.14) (width 0.406) (layer F.Cu) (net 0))
 (via (at 102.344642 110.49) (size 0.8) (drill 0.4) (layers F.Cu B.Cu) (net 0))
 (segment (start 127 102.87) (end 93.98 102.87) (width 0.406) (layer F.Cu) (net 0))
 (segment (start 128.27 106.68) (end 128.27 104.14) (width 0.406) (layer F.Cu) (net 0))
 (segment (start 128.27 104.14) (end 127 102.87) (width 0.406) (layer F.Cu) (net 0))
 (segment (start 130.81 104.14) (end 127 100.33) (width 0.406) (layer F.Cu) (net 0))
 (segment (start 127 100.33) (end 100.33 100.33) (width 0.406) (layer F.Cu) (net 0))
 (segment (start 128.27 109.22) (end 130.81 106.68) (width 0.406) (layer F.Cu) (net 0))
 (segment (start 130.81 106.68) (end 130.81 104.14) (width 0.406) (layer F.Cu) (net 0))
 (segment (start 125.73 115.57) (end 109.22 115.57) (width 0.406) (layer F.Cu) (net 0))
 (segment (start 108.349999 116.440001) (end 107.95 116.84) (width 0.406) (layer F.Cu) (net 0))
 (segment (start 109.22 115.57) (end 108.349999 116.440001) (width 0.406) (layer F.Cu) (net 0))
 (via (at 107.95 116.84) (size 0.8) (drill 0.4) (layers F.Cu B.Cu) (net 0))
 (segment (start 128.27 115.57) (end 128.27 114.3) (width 0.406) (layer F.Cu) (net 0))
 (via (at 95.25 118.11) (size 0.8) (drill 0.4) (layers F.Cu B.Cu) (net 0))
 (segment (start 125.73 118.11) (end 128.27 115.57) (width 0.406) (layer F.Cu) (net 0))
 (segment (start 95.25 118.11) (end 125.73 118.11) (width 0.406) (layer F.Cu) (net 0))
 (via (at 110.49 111.76) (size 0.8) (drill 0.4) (layers F.Cu B.Cu) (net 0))
 (segment (start 125.73 113.03) (end 111.76 113.03) (width 0.406) (layer F.Cu) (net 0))
 (segment (start 111.76 113.03) (end 110.49 111.76) (width 0.406) (layer F.Cu) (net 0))
 (segment (start 130.81 114.3) (end 128.27 111.76) (width 0.406) (layer F.Cu) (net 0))
 (segment (start 130.81 116.84) (end 130.81 114.3) (width 0.406) (layer F.Cu) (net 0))
 (segment (start 127 120.65) (end 130.81 116.84) (width 0.406) (layer F.Cu) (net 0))
 (via (at 101.6 120.65) (size 0.8) (drill 0.4) (layers F.Cu B.Cu) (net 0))
 (segment (start 101.6 120.65) (end 127 120.65) (width 0.406) (layer F.Cu) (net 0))
 (segment (start 103.614642 109.22) (end 102.344642 110.49) (width 0.406) (layer F.Cu) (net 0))
 (segment (start 125.73 110.49) (end 124.46 109.22) (width 0.406) (layer F.Cu) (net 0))
 (segment (start 124.46 109.22) (end 103.614642 109.22) (width 0.406) (layer F.Cu) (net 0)))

